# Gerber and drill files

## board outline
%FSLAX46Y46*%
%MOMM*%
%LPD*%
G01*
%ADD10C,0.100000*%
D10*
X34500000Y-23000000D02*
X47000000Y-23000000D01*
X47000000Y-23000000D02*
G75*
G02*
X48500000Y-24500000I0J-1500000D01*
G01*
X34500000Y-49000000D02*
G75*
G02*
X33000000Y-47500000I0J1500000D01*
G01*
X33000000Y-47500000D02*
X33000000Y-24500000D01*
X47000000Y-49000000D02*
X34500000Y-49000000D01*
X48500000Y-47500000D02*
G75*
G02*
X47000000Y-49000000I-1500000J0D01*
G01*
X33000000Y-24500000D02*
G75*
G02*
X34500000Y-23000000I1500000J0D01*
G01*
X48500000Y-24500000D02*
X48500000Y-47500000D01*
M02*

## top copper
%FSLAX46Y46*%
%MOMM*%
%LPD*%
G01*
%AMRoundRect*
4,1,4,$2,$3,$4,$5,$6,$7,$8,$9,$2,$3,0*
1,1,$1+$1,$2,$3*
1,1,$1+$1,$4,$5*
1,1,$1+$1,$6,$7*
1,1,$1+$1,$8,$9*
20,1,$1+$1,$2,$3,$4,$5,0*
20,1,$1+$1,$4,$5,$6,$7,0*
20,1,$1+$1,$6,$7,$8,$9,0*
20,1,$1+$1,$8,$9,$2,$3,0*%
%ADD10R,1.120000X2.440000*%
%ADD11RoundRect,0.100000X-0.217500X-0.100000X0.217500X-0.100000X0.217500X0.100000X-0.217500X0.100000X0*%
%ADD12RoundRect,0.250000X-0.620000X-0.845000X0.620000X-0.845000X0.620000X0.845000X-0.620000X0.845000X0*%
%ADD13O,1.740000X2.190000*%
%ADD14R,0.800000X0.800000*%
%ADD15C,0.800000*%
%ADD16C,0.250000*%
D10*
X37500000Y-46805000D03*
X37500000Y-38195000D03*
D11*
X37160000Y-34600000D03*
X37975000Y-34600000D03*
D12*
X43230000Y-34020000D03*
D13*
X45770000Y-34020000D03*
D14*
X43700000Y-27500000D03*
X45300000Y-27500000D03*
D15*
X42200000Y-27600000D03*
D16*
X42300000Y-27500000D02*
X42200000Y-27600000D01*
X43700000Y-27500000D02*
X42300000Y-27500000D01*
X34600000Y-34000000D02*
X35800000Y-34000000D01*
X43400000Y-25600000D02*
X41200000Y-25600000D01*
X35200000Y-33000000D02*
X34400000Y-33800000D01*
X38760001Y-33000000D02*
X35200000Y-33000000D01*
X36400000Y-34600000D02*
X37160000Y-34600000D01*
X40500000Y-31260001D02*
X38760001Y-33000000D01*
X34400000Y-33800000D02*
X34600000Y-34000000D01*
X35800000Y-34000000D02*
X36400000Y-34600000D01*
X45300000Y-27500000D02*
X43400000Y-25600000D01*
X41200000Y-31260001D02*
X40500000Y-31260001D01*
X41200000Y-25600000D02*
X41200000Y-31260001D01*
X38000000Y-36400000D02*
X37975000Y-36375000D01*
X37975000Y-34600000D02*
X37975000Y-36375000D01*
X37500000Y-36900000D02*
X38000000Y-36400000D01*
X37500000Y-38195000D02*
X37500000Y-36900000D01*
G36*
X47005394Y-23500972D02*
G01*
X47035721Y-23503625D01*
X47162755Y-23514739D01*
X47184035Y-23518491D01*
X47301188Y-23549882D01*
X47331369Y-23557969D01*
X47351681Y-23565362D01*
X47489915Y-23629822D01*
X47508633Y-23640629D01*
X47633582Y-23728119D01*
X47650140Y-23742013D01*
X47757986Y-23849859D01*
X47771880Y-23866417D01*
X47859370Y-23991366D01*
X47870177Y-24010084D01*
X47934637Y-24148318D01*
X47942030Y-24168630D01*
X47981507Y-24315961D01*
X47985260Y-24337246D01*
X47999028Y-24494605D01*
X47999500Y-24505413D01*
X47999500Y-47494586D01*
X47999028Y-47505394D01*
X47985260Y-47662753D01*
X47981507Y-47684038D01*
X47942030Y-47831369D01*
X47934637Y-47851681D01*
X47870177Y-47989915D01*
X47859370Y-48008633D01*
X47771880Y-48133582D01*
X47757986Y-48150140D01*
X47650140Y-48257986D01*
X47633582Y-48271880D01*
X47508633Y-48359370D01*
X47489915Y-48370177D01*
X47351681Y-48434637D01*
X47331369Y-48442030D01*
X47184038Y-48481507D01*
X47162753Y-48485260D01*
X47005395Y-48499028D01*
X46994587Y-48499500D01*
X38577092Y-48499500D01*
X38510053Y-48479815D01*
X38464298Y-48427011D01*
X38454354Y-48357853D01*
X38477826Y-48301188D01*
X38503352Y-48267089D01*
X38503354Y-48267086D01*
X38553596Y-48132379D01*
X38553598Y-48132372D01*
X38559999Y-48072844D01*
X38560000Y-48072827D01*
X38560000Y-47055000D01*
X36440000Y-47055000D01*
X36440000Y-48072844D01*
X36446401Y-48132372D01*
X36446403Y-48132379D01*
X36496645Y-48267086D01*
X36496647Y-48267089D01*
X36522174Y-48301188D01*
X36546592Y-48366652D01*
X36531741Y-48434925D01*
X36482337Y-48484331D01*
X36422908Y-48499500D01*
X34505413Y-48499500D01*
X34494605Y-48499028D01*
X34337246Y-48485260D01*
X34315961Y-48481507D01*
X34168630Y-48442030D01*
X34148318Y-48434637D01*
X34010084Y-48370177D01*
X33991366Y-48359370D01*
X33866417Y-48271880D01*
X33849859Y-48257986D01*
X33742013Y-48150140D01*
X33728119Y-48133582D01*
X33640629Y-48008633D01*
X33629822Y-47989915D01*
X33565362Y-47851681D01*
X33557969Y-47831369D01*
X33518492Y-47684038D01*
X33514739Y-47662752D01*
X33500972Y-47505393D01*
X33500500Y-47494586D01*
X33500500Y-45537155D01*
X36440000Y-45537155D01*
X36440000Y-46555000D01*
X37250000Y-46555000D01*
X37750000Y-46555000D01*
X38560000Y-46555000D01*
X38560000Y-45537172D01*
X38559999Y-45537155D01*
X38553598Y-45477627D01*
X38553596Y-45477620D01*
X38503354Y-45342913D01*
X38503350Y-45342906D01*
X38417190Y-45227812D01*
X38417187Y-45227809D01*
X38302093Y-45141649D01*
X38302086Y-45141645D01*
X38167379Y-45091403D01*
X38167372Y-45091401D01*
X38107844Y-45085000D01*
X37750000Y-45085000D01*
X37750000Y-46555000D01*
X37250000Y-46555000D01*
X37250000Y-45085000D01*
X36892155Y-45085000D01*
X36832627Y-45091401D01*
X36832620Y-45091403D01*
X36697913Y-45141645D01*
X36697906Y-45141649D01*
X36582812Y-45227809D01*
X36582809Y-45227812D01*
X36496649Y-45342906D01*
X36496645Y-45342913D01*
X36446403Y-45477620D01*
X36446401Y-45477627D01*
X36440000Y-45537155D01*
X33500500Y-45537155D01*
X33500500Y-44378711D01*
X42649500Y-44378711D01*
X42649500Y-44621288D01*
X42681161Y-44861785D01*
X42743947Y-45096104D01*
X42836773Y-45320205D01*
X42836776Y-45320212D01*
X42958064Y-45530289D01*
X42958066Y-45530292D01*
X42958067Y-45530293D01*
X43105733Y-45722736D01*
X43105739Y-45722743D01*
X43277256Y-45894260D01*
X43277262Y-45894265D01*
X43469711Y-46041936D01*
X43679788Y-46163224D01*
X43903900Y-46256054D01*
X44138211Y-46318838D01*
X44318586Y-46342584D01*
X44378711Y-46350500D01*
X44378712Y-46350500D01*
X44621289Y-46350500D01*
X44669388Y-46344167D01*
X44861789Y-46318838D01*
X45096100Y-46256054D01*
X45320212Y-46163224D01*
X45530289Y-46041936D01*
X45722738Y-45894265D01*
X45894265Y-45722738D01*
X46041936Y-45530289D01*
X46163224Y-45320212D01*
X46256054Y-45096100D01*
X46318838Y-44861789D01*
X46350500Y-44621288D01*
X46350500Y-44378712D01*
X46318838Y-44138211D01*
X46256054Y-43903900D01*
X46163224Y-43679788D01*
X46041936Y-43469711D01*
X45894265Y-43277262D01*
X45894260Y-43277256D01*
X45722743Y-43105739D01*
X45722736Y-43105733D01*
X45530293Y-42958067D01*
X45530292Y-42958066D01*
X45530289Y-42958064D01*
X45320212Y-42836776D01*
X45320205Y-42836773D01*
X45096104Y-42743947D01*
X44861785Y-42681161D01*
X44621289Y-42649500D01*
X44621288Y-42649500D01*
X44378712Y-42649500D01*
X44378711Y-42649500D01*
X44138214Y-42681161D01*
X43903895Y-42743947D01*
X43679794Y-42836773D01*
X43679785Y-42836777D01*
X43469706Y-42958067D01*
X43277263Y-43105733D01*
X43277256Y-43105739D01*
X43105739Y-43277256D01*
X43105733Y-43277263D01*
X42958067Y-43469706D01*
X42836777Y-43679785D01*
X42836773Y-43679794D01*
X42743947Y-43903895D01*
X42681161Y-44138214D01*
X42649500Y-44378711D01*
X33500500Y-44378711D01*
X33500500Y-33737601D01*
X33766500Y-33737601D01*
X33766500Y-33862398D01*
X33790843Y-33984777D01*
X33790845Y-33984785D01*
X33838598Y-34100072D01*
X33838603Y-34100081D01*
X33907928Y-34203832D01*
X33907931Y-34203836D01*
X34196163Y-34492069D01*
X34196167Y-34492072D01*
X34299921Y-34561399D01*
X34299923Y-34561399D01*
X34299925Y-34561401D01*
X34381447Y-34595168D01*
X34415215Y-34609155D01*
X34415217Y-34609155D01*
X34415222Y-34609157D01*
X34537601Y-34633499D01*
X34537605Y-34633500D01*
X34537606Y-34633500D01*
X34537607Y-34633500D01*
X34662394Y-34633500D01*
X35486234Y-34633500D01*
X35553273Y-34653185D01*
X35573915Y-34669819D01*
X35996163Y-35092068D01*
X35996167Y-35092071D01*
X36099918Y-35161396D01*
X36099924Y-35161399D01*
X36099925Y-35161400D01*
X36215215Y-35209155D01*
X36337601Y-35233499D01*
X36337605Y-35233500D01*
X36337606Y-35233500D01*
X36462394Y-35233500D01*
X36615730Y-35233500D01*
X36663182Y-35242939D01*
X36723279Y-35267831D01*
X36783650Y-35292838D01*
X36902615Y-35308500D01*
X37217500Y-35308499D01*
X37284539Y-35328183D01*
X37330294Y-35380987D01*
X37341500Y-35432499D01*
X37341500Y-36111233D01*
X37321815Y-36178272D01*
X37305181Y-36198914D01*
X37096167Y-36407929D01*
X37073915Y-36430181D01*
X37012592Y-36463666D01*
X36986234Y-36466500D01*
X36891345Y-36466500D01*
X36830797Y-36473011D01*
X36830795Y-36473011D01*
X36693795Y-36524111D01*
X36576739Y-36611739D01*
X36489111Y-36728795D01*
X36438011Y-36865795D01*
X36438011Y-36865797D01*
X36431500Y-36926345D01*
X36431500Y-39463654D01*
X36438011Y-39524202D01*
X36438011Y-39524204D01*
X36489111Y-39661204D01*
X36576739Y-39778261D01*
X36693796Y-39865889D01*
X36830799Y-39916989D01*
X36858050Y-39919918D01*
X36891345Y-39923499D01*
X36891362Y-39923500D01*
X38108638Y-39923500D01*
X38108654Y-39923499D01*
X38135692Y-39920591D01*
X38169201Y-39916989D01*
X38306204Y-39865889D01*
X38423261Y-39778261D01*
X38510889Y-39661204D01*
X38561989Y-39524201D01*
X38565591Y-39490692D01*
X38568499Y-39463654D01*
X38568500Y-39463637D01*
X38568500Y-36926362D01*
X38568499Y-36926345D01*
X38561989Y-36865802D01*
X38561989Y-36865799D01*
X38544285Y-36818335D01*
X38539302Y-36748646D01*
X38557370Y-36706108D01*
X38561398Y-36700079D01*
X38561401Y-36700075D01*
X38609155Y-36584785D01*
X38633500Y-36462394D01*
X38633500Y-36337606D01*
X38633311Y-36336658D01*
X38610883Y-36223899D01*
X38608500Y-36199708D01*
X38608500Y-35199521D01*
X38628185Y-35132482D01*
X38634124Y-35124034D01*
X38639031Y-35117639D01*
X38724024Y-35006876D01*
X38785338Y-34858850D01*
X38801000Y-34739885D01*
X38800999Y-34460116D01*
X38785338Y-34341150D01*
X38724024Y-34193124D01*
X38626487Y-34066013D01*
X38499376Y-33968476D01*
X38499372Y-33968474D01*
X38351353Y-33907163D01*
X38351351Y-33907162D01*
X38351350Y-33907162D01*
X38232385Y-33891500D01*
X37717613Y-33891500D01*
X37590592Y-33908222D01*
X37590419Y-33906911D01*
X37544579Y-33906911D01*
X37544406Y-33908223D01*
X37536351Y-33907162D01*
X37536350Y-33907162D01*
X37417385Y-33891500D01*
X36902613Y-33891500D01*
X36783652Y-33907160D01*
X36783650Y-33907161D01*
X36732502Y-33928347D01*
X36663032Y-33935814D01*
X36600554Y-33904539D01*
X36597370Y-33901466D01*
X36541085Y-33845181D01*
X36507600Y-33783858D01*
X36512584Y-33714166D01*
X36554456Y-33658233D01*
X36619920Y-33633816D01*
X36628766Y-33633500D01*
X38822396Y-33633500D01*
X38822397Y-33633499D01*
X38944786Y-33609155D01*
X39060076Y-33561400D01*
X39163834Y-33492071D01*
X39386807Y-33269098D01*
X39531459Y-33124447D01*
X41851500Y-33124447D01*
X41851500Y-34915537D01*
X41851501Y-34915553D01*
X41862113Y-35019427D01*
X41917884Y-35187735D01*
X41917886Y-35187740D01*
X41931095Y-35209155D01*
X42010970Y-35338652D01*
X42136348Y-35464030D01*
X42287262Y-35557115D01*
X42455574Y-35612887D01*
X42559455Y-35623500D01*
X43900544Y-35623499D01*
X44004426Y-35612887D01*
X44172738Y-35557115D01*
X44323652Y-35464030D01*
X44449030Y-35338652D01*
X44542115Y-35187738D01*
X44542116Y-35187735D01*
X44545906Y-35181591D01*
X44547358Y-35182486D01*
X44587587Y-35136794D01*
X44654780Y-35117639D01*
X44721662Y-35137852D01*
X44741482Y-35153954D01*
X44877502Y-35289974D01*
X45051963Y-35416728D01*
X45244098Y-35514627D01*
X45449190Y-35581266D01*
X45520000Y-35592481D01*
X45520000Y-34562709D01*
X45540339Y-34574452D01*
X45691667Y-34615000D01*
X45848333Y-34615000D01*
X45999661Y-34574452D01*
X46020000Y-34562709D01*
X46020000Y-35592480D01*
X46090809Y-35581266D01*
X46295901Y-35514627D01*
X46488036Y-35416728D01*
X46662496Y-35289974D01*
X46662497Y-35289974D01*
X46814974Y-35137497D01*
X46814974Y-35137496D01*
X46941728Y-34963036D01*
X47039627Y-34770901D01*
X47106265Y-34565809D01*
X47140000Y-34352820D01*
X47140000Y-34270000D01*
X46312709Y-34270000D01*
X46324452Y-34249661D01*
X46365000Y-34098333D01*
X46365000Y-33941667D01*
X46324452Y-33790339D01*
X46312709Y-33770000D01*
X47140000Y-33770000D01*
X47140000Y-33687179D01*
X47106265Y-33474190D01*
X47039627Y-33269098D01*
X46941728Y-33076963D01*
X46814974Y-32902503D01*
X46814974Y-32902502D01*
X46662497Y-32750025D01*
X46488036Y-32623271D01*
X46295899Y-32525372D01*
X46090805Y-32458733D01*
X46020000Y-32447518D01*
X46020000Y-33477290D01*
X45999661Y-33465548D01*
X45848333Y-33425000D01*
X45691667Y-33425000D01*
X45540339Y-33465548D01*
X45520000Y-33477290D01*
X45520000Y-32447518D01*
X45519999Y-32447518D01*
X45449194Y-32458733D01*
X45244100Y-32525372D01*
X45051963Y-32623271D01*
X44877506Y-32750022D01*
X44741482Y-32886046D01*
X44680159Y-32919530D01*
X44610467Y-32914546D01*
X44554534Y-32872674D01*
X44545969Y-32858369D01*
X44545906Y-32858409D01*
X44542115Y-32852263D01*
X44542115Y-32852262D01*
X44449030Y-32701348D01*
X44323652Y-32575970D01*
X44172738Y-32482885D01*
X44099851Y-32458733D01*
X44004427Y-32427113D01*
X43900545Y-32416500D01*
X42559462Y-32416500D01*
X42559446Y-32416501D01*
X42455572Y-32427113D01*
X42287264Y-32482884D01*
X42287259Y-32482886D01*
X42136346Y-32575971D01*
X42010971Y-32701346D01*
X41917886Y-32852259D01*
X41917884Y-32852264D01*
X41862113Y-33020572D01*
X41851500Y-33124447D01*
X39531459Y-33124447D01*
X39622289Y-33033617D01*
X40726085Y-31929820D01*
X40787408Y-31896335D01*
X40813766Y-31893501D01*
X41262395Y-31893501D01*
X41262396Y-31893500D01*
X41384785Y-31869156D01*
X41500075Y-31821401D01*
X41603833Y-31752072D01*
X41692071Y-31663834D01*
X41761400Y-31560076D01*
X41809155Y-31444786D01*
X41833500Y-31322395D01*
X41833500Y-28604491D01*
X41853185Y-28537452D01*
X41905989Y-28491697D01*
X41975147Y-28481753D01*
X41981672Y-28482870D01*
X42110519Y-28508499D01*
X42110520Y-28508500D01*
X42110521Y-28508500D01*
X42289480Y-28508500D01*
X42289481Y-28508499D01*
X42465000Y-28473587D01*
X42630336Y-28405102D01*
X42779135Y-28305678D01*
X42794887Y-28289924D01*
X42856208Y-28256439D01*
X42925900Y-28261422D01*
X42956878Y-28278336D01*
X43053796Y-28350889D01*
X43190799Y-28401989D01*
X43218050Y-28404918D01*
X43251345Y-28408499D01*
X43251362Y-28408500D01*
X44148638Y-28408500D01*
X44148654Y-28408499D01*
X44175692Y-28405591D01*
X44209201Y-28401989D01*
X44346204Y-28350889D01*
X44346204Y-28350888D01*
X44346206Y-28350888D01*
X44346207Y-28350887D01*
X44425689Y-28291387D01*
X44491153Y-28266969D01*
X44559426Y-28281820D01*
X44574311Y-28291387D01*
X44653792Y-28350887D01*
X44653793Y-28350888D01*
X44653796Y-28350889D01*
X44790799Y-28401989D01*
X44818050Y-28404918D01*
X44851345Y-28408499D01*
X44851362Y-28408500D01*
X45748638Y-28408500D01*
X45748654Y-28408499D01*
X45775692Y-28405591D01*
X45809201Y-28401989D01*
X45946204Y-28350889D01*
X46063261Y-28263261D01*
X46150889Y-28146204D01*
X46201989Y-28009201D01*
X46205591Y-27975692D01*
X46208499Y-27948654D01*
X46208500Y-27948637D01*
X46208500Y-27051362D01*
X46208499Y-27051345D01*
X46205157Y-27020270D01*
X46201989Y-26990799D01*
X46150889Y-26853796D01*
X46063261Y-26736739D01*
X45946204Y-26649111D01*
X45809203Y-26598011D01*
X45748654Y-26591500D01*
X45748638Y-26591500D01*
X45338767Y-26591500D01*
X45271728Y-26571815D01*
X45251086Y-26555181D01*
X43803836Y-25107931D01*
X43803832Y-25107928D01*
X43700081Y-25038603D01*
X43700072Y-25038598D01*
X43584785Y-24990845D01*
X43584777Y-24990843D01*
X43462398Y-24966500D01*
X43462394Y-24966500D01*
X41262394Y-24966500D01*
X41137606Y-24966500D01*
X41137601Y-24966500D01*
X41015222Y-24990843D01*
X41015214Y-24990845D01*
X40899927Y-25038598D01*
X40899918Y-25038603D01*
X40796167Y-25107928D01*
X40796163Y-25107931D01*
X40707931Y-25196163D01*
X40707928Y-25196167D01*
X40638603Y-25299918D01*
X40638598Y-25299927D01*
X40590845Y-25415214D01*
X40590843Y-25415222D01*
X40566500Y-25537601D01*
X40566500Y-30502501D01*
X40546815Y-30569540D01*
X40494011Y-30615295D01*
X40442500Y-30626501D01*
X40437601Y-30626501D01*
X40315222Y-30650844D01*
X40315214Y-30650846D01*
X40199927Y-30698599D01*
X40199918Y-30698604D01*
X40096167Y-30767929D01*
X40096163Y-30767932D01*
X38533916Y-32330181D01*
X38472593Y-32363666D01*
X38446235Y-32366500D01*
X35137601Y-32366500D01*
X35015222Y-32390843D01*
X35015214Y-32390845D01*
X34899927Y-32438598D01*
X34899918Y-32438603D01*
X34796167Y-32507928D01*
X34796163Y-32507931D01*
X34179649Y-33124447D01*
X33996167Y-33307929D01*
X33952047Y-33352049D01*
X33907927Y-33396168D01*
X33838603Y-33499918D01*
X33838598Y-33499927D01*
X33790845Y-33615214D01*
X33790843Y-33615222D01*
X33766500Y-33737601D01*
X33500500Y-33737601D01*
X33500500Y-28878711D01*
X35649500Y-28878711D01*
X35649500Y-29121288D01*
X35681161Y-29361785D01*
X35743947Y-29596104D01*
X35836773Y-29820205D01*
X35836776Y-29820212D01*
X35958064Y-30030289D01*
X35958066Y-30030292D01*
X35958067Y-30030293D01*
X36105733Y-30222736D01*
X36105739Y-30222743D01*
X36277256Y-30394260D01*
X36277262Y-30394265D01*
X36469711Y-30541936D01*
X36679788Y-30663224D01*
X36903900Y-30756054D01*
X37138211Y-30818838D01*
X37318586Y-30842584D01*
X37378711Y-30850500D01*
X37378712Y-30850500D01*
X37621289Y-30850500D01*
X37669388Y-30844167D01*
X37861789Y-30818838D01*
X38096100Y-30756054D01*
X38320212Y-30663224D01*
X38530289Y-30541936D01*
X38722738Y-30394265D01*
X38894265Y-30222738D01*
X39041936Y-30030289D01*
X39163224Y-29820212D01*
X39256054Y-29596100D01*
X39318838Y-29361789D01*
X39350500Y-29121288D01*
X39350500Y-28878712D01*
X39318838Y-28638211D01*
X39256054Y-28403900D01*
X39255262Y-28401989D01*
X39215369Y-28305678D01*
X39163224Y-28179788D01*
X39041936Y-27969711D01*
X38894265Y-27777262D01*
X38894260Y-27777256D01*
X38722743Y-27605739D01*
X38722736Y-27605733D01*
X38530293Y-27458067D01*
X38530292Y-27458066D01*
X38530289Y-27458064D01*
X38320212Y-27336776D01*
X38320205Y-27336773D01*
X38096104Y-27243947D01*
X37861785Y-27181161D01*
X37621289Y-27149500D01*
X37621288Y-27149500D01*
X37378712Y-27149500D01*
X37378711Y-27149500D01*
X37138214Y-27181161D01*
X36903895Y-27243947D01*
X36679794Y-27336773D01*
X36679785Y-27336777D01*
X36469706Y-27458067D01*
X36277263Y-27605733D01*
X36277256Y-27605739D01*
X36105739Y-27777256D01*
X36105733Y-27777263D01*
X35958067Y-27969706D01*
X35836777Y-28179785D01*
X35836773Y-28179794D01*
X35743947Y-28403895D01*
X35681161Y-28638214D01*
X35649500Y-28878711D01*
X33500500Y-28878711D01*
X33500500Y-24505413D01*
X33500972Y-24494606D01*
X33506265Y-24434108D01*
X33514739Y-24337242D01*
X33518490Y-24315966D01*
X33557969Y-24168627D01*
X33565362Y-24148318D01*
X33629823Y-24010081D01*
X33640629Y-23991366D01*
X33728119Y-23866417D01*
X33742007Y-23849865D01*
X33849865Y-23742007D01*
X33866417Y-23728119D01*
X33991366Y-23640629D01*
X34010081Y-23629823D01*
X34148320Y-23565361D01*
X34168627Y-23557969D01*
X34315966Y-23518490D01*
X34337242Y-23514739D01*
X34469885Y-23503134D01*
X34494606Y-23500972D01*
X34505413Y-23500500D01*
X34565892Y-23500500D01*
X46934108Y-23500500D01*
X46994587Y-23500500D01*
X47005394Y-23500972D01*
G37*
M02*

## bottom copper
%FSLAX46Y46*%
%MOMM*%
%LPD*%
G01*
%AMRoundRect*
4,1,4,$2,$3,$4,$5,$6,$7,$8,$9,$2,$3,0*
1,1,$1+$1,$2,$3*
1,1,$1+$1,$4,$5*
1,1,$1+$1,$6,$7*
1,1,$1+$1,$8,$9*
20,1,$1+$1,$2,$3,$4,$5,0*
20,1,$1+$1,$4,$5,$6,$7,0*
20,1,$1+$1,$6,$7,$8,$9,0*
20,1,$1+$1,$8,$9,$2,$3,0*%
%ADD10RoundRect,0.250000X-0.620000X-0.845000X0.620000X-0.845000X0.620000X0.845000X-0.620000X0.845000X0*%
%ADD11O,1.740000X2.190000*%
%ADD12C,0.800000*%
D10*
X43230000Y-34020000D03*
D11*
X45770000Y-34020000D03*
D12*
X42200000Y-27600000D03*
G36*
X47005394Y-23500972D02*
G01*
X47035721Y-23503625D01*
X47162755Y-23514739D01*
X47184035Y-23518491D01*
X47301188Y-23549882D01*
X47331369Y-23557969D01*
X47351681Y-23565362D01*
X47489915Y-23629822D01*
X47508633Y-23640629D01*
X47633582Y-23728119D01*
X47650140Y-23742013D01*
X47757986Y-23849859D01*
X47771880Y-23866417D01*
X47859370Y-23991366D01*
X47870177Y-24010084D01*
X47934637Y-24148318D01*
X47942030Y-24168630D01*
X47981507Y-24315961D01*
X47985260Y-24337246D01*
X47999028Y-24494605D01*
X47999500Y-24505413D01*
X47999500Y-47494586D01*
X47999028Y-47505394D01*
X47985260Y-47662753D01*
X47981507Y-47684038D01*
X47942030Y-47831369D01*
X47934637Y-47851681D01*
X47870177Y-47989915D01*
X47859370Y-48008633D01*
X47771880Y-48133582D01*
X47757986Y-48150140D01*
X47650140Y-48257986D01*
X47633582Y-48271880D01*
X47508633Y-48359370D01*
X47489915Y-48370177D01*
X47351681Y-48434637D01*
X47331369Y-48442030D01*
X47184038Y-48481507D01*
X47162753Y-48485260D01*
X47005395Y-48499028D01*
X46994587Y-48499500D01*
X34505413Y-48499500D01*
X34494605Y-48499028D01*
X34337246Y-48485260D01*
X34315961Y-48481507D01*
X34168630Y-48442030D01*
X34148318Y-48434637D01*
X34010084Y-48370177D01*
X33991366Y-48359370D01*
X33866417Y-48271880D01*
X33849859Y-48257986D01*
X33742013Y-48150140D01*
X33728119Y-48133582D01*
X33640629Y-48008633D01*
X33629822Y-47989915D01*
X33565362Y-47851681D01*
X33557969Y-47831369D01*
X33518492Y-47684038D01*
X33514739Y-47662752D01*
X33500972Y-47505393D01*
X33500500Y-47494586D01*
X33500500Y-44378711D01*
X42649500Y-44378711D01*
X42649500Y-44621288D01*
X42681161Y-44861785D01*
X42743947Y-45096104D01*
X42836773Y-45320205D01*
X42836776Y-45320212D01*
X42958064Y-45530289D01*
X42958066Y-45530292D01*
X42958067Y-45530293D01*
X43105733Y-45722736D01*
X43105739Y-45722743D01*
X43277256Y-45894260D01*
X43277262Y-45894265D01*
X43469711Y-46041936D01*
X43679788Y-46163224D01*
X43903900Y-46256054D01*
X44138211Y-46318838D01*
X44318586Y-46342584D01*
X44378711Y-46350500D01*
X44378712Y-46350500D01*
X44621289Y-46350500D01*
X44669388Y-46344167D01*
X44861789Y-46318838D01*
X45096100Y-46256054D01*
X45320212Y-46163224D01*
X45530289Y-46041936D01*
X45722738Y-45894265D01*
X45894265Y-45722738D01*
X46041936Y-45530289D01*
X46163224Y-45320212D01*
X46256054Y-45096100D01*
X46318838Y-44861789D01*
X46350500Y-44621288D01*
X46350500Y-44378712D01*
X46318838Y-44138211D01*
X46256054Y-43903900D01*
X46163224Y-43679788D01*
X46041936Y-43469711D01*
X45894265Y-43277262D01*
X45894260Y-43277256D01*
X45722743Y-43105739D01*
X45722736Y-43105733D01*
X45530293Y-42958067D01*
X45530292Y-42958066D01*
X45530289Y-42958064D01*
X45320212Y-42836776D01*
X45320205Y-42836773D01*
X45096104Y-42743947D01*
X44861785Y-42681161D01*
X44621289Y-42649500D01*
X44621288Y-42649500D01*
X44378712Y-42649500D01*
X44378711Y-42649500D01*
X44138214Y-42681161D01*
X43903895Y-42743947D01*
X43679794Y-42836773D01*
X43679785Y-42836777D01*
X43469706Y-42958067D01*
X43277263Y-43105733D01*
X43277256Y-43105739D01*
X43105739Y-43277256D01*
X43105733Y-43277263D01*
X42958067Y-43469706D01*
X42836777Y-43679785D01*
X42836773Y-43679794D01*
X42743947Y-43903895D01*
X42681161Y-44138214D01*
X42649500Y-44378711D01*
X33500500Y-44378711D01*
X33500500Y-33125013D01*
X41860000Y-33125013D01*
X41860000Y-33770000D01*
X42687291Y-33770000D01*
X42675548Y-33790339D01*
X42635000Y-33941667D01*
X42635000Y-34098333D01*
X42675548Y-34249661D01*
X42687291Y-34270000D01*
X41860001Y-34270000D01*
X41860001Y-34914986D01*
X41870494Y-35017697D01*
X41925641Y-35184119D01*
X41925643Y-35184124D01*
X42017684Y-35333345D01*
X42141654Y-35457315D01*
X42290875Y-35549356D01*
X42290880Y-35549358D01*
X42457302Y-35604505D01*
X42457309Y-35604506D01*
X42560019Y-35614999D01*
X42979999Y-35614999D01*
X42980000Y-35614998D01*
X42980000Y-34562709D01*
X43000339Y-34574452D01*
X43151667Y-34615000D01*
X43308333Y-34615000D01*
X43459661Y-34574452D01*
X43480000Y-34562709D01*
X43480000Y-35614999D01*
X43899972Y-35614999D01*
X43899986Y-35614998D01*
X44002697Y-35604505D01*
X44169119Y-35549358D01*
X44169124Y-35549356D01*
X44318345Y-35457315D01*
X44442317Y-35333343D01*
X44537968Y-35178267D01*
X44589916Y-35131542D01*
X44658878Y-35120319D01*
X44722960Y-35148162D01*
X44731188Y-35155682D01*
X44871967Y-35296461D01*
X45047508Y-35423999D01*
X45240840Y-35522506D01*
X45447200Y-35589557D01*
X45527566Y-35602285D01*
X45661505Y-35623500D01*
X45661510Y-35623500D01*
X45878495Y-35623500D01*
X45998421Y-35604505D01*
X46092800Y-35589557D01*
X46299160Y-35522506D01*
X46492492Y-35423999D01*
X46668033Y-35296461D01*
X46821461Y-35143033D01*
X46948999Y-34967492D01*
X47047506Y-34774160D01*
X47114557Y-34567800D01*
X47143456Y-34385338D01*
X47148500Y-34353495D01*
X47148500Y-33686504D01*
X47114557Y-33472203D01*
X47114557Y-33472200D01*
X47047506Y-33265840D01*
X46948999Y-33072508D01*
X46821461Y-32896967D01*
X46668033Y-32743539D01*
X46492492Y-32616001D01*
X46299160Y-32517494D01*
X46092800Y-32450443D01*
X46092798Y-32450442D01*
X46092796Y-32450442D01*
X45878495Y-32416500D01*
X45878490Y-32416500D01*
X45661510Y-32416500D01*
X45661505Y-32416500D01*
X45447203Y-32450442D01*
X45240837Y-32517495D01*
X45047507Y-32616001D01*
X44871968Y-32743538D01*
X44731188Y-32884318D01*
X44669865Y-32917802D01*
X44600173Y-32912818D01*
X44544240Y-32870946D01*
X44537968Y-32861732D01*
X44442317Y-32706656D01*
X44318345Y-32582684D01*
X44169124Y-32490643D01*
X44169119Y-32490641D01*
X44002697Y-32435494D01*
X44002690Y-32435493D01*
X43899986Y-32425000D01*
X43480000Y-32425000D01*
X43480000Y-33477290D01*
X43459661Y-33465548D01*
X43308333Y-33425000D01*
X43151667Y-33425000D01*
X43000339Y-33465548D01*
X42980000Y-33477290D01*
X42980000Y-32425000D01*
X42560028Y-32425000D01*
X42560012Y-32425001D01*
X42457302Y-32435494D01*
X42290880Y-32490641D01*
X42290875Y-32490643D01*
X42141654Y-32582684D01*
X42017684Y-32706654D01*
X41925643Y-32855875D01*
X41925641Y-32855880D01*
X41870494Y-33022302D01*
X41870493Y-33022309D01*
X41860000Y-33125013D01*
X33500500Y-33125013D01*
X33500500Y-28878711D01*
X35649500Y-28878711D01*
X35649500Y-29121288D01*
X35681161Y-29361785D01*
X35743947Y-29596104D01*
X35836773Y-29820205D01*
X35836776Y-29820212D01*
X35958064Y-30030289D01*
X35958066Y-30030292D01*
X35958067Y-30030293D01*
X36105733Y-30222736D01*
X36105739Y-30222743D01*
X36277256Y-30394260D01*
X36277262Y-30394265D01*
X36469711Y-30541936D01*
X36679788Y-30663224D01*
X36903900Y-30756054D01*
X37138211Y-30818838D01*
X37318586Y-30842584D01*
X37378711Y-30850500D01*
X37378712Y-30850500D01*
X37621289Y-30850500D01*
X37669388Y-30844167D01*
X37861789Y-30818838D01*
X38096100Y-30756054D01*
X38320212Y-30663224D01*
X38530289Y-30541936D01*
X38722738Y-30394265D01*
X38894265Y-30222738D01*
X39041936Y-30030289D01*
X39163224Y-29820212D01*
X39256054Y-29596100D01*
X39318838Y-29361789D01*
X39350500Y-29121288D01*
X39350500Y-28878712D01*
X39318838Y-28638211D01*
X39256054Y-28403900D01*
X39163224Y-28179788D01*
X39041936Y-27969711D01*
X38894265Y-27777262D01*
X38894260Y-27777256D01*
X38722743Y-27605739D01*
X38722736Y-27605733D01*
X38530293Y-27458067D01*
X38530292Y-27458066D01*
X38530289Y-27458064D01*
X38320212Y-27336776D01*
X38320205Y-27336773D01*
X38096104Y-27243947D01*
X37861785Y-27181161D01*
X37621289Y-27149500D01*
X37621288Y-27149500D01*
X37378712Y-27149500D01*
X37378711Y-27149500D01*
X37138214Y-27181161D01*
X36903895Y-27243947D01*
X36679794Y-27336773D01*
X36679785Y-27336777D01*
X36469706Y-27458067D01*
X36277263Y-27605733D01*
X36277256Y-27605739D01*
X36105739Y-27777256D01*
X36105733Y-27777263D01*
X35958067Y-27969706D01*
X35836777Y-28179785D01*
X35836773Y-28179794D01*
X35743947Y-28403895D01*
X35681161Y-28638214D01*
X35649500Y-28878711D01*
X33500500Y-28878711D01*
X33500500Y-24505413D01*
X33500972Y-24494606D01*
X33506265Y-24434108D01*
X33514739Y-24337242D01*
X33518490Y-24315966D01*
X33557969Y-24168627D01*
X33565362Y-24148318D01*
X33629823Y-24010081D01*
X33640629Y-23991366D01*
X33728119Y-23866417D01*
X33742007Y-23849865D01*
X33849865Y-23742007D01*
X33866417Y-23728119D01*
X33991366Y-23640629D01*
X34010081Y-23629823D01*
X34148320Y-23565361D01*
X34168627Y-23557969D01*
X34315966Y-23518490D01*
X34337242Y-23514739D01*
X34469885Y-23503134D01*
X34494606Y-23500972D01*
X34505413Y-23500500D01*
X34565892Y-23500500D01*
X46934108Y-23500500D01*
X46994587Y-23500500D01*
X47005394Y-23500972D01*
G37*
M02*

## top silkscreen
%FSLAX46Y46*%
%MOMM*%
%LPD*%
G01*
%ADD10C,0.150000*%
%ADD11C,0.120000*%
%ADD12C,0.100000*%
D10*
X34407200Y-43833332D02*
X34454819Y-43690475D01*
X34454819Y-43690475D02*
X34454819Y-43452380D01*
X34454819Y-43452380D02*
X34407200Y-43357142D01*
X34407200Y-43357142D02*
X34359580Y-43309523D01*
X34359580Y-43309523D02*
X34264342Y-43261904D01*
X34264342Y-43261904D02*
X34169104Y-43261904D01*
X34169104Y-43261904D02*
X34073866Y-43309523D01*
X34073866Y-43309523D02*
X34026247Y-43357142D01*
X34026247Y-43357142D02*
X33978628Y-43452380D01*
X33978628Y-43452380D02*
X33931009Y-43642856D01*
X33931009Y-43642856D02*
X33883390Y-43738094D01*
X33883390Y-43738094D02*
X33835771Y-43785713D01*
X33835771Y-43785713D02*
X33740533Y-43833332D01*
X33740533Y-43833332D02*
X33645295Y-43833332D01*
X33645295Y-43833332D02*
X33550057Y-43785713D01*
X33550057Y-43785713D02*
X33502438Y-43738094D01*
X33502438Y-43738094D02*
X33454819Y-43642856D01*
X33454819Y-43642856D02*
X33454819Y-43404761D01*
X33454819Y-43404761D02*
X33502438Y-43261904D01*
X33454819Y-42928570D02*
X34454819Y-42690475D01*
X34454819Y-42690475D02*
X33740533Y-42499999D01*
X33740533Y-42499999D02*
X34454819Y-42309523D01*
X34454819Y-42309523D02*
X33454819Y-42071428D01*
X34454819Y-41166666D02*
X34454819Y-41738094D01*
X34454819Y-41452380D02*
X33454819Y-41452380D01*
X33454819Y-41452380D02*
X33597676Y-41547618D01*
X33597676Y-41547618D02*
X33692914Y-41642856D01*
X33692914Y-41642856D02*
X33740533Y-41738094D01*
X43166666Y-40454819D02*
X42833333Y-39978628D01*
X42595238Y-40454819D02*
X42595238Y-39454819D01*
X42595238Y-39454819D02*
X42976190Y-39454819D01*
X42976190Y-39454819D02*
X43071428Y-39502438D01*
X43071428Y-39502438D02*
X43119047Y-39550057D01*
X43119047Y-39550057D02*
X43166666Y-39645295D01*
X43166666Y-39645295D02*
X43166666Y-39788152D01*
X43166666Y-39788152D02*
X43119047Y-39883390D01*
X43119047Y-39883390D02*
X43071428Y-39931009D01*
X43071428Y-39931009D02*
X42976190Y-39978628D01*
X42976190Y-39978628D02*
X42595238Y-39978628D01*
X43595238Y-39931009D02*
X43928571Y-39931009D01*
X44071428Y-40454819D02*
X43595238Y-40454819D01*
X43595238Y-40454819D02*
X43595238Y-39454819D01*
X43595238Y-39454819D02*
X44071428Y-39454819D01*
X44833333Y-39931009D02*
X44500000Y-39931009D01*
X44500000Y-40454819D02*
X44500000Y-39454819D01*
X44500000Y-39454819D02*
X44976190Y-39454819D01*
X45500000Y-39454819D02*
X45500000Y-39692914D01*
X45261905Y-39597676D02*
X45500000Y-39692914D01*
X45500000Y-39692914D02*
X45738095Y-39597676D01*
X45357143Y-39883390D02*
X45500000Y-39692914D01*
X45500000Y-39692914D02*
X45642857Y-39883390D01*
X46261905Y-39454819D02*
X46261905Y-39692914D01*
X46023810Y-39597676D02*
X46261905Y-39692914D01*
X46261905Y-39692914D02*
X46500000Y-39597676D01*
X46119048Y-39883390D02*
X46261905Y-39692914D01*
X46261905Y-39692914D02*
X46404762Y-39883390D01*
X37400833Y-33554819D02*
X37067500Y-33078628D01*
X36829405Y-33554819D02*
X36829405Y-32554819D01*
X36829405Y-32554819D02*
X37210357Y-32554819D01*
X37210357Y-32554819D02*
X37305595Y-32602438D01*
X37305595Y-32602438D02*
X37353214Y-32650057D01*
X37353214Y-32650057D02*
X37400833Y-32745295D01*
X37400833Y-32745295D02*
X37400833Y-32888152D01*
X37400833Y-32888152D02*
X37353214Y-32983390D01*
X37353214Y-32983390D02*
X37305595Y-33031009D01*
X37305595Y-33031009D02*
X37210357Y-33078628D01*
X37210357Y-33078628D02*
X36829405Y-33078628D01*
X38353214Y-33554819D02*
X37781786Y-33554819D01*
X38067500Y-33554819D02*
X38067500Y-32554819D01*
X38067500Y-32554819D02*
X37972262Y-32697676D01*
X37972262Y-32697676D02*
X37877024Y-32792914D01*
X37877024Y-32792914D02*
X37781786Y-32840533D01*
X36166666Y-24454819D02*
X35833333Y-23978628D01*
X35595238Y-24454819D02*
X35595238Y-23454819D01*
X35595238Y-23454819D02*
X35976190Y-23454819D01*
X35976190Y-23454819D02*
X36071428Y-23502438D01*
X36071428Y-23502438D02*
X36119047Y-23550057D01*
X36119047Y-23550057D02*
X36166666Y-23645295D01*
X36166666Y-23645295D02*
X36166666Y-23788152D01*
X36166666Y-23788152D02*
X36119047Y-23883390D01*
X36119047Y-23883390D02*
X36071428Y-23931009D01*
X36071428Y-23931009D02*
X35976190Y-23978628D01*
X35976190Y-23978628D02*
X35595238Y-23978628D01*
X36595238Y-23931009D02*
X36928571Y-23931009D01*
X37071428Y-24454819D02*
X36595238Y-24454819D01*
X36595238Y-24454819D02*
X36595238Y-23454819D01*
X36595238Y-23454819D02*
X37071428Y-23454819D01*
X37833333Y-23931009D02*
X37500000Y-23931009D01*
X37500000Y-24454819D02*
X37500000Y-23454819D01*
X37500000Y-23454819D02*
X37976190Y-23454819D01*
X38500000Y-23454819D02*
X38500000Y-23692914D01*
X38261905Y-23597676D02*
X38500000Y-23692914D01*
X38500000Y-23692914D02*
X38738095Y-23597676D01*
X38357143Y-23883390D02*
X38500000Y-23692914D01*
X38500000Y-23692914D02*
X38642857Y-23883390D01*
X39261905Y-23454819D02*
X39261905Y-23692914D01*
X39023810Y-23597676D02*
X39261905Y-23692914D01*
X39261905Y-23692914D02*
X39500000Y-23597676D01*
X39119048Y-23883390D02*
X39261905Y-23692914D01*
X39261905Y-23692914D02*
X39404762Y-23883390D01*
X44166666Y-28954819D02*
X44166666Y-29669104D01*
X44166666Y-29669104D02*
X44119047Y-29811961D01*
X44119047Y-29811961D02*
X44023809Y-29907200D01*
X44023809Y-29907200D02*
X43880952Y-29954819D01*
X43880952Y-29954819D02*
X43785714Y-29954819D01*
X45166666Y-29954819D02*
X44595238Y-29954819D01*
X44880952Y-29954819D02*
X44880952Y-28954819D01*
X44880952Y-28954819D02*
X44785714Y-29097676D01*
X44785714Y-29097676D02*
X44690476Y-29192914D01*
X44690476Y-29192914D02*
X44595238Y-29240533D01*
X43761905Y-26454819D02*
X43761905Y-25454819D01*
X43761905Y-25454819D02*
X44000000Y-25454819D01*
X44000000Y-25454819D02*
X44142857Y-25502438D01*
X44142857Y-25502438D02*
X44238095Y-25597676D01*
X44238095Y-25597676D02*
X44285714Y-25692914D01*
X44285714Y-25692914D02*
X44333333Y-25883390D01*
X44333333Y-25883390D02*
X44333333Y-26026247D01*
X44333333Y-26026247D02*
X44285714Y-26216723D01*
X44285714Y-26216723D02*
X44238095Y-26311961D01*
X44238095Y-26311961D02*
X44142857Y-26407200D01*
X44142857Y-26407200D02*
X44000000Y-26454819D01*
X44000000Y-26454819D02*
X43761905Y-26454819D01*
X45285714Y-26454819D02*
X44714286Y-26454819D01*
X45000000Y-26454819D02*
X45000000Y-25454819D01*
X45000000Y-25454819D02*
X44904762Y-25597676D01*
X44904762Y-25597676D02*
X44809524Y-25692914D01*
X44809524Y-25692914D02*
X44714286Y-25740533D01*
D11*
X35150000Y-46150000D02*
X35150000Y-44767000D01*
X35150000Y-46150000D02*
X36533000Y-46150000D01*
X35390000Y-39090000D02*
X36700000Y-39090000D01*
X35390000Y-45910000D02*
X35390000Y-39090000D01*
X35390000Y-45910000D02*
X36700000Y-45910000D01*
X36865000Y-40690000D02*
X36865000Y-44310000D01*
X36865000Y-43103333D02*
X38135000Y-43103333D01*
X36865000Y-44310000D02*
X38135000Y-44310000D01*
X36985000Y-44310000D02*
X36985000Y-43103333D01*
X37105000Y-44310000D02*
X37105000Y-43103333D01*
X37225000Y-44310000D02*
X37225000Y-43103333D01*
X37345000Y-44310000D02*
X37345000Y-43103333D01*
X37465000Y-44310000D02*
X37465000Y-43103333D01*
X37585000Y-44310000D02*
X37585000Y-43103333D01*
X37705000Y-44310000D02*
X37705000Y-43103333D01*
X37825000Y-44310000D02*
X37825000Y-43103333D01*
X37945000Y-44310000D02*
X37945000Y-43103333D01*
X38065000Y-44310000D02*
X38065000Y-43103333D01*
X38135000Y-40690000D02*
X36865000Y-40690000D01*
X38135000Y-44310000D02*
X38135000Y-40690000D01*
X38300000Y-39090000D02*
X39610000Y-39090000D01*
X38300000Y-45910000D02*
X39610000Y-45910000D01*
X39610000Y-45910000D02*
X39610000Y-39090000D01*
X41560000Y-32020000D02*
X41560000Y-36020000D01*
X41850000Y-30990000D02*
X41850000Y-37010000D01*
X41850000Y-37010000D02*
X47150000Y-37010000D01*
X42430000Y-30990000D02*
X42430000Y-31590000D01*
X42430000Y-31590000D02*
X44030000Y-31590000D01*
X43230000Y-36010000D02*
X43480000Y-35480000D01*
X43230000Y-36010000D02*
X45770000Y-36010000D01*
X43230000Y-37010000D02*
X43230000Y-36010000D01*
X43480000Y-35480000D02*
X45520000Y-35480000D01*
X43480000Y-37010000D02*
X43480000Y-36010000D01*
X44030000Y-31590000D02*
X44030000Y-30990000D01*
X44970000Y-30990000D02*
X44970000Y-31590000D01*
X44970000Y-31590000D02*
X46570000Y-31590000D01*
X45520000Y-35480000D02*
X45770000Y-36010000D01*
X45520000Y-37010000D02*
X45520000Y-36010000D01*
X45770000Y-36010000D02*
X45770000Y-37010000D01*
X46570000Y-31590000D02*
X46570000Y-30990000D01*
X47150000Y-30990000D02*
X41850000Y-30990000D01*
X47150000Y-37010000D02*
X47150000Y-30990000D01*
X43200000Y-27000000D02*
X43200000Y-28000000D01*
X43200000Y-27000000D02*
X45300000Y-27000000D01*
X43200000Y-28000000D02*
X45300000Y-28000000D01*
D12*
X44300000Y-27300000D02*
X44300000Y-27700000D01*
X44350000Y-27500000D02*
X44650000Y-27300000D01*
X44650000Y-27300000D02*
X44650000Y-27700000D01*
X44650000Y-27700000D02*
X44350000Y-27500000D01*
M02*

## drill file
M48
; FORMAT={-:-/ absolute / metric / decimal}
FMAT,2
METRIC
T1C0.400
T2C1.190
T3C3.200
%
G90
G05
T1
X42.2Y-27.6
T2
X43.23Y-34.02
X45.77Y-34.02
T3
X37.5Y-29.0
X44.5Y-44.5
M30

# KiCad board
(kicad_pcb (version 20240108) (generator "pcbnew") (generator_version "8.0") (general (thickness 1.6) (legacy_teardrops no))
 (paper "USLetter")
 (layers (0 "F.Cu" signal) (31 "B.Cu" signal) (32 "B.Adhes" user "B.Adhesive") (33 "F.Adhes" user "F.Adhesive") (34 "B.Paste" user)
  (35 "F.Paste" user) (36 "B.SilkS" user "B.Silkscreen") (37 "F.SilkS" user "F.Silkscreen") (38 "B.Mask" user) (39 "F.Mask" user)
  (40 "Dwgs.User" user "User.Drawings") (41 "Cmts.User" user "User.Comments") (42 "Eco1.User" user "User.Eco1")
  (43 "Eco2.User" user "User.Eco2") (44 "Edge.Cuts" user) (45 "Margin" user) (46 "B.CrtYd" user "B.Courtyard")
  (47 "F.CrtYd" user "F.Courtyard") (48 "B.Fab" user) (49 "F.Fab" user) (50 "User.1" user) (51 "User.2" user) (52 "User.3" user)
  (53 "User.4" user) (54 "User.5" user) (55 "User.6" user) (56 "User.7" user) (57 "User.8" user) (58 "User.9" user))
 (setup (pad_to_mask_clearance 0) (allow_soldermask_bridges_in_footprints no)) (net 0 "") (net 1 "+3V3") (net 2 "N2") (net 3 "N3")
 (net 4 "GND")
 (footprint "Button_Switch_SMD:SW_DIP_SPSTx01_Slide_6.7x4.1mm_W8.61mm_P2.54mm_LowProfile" (layer "F.Cu") (at 37.5 42.5 90)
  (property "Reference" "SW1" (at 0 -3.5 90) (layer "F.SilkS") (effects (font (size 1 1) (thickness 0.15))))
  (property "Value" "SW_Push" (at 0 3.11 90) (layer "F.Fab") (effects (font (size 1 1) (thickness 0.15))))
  (fp_line (start -3.65 -2.35) (end -2.267 -2.35) (stroke (width 0.12) (type solid)) (layer "F.SilkS"))
  (fp_line (start -3.65 -2.35) (end -3.65 -0.967) (stroke (width 0.12) (type solid)) (layer "F.SilkS"))
  (fp_line (start 3.41 -2.11) (end 3.41 -0.8) (stroke (width 0.12) (type solid)) (layer "F.SilkS"))
  (fp_line (start -3.41 -2.11) (end 3.41 -2.11) (stroke (width 0.12) (type solid)) (layer "F.SilkS"))
  (fp_line (start -3.41 -2.11) (end -3.41 -0.8) (stroke (width 0.12) (type solid)) (layer "F.SilkS"))
  (fp_line (start 1.81 -0.635) (end -1.81 -0.635) (stroke (width 0.12) (type solid)) (layer "F.SilkS"))
  (fp_line (start -0.603333 -0.635) (end -0.603333 0.635) (stroke (width 0.12) (type solid)) (layer "F.SilkS"))
  (fp_line (start -1.81 -0.635) (end -1.81 0.635) (stroke (width 0.12) (type solid)) (layer "F.SilkS"))
  (fp_line (start -1.81 -0.515) (end -0.603333 -0.515) (stroke (width 0.12) (type solid)) (layer "F.SilkS"))
  (fp_line (start -1.81 -0.395) (end -0.603333 -0.395) (stroke (width 0.12) (type solid)) (layer "F.SilkS"))
  (fp_line (start -1.81 -0.275) (end -0.603333 -0.275) (stroke (width 0.12) (type solid)) (layer "F.SilkS"))
  (fp_line (start -1.81 -0.155) (end -0.603333 -0.155) (stroke (width 0.12) (type solid)) (layer "F.SilkS"))
  (fp_line (start -1.81 -0.035) (end -0.603333 -0.035) (stroke (width 0.12) (type solid)) (layer "F.SilkS"))
  (fp_line (start -1.81 0.085) (end -0.603333 0.085) (stroke (width 0.12) (type solid)) (layer "F.SilkS"))
  (fp_line (start -1.81 0.205) (end -0.603333 0.205) (stroke (width 0.12) (type solid)) (layer "F.SilkS"))
  (fp_line (start -1.81 0.325) (end -0.603333 0.325) (stroke (width 0.12) (type solid)) (layer "F.SilkS"))
  (fp_line (start -1.81 0.445) (end -0.603333 0.445) (stroke (width 0.12) (type solid)) (layer "F.SilkS"))
  (fp_line (start -1.81 0.565) (end -0.603333 0.565) (stroke (width 0.12) (type solid)) (layer "F.SilkS"))
  (fp_line (start 1.81 0.635) (end 1.81 -0.635) (stroke (width 0.12) (type solid)) (layer "F.SilkS"))
  (fp_line (start -1.81 0.635) (end 1.81 0.635) (stroke (width 0.12) (type solid)) (layer "F.SilkS"))
  (fp_line (start 3.41 0.8) (end 3.41 2.11) (stroke (width 0.12) (type solid)) (layer "F.SilkS"))
  (fp_line (start -3.41 0.8) (end -3.41 2.11) (stroke (width 0.12) (type solid)) (layer "F.SilkS"))
  (fp_line (start -3.41 2.11) (end 3.41 2.11) (stroke (width 0.12) (type solid)) (layer "F.SilkS"))
  (pad "1" smd rect (at -4.305 0 90) (size 2.44 1.12) (layers "F.Cu" "F.Paste" "F.Mask") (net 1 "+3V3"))
  (pad "2" smd rect (at 4.305 0 90) (size 2.44 1.12) (layers "F.Cu" "F.Paste" "F.Mask") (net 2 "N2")))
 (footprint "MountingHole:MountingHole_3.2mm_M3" (layer "F.Cu") (at 44.5 44.5)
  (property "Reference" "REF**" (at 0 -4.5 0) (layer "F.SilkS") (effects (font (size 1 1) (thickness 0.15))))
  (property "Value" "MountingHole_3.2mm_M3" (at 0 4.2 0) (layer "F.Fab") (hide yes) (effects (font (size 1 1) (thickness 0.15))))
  (pad "" np_thru_hole circle (at 0 0) (size 3.2 3.2) (drill 3.2) (layers "*.Cu" "*.Mask")))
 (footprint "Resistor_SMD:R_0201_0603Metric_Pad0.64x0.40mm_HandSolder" (layer "F.Cu") (at 37.5675 34.6)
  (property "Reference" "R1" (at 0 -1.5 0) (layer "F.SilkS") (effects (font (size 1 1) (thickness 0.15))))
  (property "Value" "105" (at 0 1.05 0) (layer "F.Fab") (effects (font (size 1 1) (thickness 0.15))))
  (pad "" smd roundrect (at -0.4325 0) (size 0.458 0.36) (layers "F.Paste") (roundrect_rratio 0.25))
  (pad "" smd roundrect (at 0.4325 0) (size 0.458 0.36) (layers "F.Paste") (roundrect_rratio 0.25))
  (pad "1" smd roundrect (at -0.4075 0) (size 0.635 0.4) (layers "F.Cu" "F.Mask") (roundrect_rratio 0.25) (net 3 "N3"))
  (pad "2" smd roundrect (at 0.4075 0) (size 0.635 0.4) (layers "F.Cu" "F.Mask") (roundrect_rratio 0.25) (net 2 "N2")))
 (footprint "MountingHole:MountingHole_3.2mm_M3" (layer "F.Cu") (at 37.5 29)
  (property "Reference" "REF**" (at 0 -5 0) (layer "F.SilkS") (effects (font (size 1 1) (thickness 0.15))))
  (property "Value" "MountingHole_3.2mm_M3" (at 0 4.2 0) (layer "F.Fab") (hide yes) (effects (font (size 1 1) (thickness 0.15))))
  (pad "" np_thru_hole circle (at 0 0) (size 3.2 3.2) (drill 3.2) (layers "*.Cu" "*.Mask")))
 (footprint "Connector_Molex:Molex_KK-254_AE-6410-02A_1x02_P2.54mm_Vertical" (layer "F.Cu") (at 43.23 34.02)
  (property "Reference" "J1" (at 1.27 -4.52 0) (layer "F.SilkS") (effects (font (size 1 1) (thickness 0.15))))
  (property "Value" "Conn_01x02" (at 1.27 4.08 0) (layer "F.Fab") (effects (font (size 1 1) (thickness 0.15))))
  (fp_line (start -1.67 -2) (end -1.67 2) (stroke (width 0.12) (type solid)) (layer "F.SilkS"))
  (fp_line (start -1.38 -3.03) (end -1.38 2.99) (stroke (width 0.12) (type solid)) (layer "F.SilkS"))
  (fp_line (start -1.38 2.99) (end 3.92 2.99) (stroke (width 0.12) (type solid)) (layer "F.SilkS"))
  (fp_line (start -0.8 -3.03) (end -0.8 -2.43) (stroke (width 0.12) (type solid)) (layer "F.SilkS"))
  (fp_line (start -0.8 -2.43) (end 0.8 -2.43) (stroke (width 0.12) (type solid)) (layer "F.SilkS"))
  (fp_line (start 0 1.99) (end 0.25 1.46) (stroke (width 0.12) (type solid)) (layer "F.SilkS"))
  (fp_line (start 0 1.99) (end 2.54 1.99) (stroke (width 0.12) (type solid)) (layer "F.SilkS"))
  (fp_line (start 0 2.99) (end 0 1.99) (stroke (width 0.12) (type solid)) (layer "F.SilkS"))
  (fp_line (start 0.25 1.46) (end 2.29 1.46) (stroke (width 0.12) (type solid)) (layer "F.SilkS"))
  (fp_line (start 0.25 2.99) (end 0.25 1.99) (stroke (width 0.12) (type solid)) (layer "F.SilkS"))
  (fp_line (start 0.8 -2.43) (end 0.8 -3.03) (stroke (width 0.12) (type solid)) (layer "F.SilkS"))
  (fp_line (start 1.74 -3.03) (end 1.74 -2.43) (stroke (width 0.12) (type solid)) (layer "F.SilkS"))
  (fp_line (start 1.74 -2.43) (end 3.34 -2.43) (stroke (width 0.12) (type solid)) (layer "F.SilkS"))
  (fp_line (start 2.29 1.46) (end 2.54 1.99) (stroke (width 0.12) (type solid)) (layer "F.SilkS"))
  (fp_line (start 2.29 2.99) (end 2.29 1.99) (stroke (width 0.12) (type solid)) (layer "F.SilkS"))
  (fp_line (start 2.54 1.99) (end 2.54 2.99) (stroke (width 0.12) (type solid)) (layer "F.SilkS"))
  (fp_line (start 3.34 -2.43) (end 3.34 -3.03) (stroke (width 0.12) (type solid)) (layer "F.SilkS"))
  (fp_line (start 3.92 -3.03) (end -1.38 -3.03) (stroke (width 0.12) (type solid)) (layer "F.SilkS"))
  (fp_line (start 3.92 2.99) (end 3.92 -3.03) (stroke (width 0.12) (type solid)) (layer "F.SilkS"))
  (pad "1" thru_hole roundrect (at 0 0) (size 1.74 2.19) (drill 1.19) (layers "*.Cu" "*.Mask") (remove_unused_layers no)
   (roundrect_rratio 0.143678) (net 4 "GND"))
  (pad "2" thru_hole oval (at 2.54 0) (size 1.74 2.19) (drill 1.19) (layers "*.Cu" "*.Mask") (remove_unused_layers no) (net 1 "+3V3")))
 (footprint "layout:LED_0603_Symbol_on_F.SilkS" (layer "F.Cu") (at 44.5 27.5)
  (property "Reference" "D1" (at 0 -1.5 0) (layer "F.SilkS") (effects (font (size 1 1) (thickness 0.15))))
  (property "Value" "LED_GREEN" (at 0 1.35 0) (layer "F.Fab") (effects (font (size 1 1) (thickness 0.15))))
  (fp_line (start -1.3 -0.5) (end -1.3 0.5) (stroke (width 0.12) (type solid)) (layer "F.SilkS"))
  (fp_line (start -1.3 -0.5) (end 0.8 -0.5) (stroke (width 0.12) (type solid)) (layer "F.SilkS"))
  (fp_line (start -1.3 0.5) (end 0.8 0.5) (stroke (width 0.12) (type solid)) (layer "F.SilkS"))
  (fp_line (start -0.2 -0.2) (end -0.2 0.2) (stroke (width 0.1) (type solid)) (layer "F.SilkS"))
  (fp_line (start -0.15 0) (end 0.15 -0.2) (stroke (width 0.1) (type solid)) (layer "F.SilkS"))
  (fp_line (start 0.15 -0.2) (end 0.15 0.2) (stroke (width 0.1) (type solid)) (layer "F.SilkS"))
  (fp_line (start 0.15 0.2) (end -0.15 0) (stroke (width 0.1) (type solid)) (layer "F.SilkS"))
  (pad "1" smd rect (at -0.8 0 180) (size 0.8 0.8) (layers "F.Cu" "F.Paste" "F.Mask") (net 4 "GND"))
  (pad "2" smd rect (at 0.8 0 180) (size 0.8 0.8) (layers "F.Cu" "F.Paste" "F.Mask") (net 3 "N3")))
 (gr_line (start 34.5 23) (end 47 23) (stroke (width 0.1) (type default)) (layer "Edge.Cuts"))
 (gr_arc (start 47 23) (mid 48.06066 23.43934) (end 48.5 24.5) (stroke (width 0.1) (type default)) (layer "Edge.Cuts"))
 (gr_arc (start 34.5 49) (mid 33.43934 48.56066) (end 33 47.5) (stroke (width 0.1) (type default)) (layer "Edge.Cuts"))
 (gr_line (start 33 47.5) (end 33 24.5) (stroke (width 0.1) (type default)) (layer "Edge.Cuts"))
 (gr_line (start 47 49) (end 34.5 49) (stroke (width 0.1) (type default)) (layer "Edge.Cuts"))
 (gr_arc (start 48.5 47.5) (mid 48.06066 48.56066) (end 47 49) (stroke (width 0.1) (type default)) (layer "Edge.Cuts"))
 (gr_arc (start 33 24.5) (mid 33.43934 23.43934) (end 34.5 23) (stroke (width 0.1) (type default)) (layer "Edge.Cuts"))
 (gr_line (start 48.5 24.5) (end 48.5 47.5) (stroke (width 0.1) (type default)) (layer "Edge.Cuts"))
 (segment (start 42.3 27.5) (end 42.2 27.6) (width 0.25) (layer "F.Cu") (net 4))
 (segment (start 43.7 27.5) (end 42.3 27.5) (width 0.25) (layer "F.Cu") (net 4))
 (via (at 42.2 27.6) (size 0.8) (drill 0.4) (layers "F.Cu" "B.Cu") (free yes) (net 4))
 (segment (start 34.6 34) (end 35.8 34) (width 0.25) (layer "F.Cu") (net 3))
 (segment (start 43.4 25.6) (end 41.2 25.6) (width 0.25) (layer "F.Cu") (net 3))
 (segment (start 35.2 33) (end 34.4 33.8) (width 0.25) (layer "F.Cu") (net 3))
 (segment (start 38.760001 33) (end 35.2 33) (width 0.25) (layer "F.Cu") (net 3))
 (segment (start 36.4 34.6) (end 37.16 34.6) (width 0.25) (layer "F.Cu") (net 3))
 (segment (start 40.5 31.260001) (end 38.760001 33) (width 0.25) (layer "F.Cu") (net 3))
 (segment (start 34.4 33.8) (end 34.6 34) (width 0.25) (layer "F.Cu") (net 3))
 (segment (start 35.8 34) (end 36.4 34.6) (width 0.25) (layer "F.Cu") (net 3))
 (segment (start 45.3 27.5) (end 43.4 25.6) (width 0.25) (layer "F.Cu") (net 3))
 (segment (start 41.2 31.260001) (end 40.5 31.260001) (width 0.25) (layer "F.Cu") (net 3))
 (segment (start 41.2 25.6) (end 41.2 31.260001) (width 0.25) (layer "F.Cu") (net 3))
 (segment (start 38 36.4) (end 37.975 36.375) (width 0.25) (layer "F.Cu") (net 2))
 (segment (start 37.975 34.6) (end 37.975 36.375) (width 0.25) (layer "F.Cu") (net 2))
 (segment (start 37.5 36.9) (end 38 36.4) (width 0.25) (layer "F.Cu") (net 2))
 (segment (start 37.5 38.195) (end 37.5 36.9) (width 0.25) (layer "F.Cu") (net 2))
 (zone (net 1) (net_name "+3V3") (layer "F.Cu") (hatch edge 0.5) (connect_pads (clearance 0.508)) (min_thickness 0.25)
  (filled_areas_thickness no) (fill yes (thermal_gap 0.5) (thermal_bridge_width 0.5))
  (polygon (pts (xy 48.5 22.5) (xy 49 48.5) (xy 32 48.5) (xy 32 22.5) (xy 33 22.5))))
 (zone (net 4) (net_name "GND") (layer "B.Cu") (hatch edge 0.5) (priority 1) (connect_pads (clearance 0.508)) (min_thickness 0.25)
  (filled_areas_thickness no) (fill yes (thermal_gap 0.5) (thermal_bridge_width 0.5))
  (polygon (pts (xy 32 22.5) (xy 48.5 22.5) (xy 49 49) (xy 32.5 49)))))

